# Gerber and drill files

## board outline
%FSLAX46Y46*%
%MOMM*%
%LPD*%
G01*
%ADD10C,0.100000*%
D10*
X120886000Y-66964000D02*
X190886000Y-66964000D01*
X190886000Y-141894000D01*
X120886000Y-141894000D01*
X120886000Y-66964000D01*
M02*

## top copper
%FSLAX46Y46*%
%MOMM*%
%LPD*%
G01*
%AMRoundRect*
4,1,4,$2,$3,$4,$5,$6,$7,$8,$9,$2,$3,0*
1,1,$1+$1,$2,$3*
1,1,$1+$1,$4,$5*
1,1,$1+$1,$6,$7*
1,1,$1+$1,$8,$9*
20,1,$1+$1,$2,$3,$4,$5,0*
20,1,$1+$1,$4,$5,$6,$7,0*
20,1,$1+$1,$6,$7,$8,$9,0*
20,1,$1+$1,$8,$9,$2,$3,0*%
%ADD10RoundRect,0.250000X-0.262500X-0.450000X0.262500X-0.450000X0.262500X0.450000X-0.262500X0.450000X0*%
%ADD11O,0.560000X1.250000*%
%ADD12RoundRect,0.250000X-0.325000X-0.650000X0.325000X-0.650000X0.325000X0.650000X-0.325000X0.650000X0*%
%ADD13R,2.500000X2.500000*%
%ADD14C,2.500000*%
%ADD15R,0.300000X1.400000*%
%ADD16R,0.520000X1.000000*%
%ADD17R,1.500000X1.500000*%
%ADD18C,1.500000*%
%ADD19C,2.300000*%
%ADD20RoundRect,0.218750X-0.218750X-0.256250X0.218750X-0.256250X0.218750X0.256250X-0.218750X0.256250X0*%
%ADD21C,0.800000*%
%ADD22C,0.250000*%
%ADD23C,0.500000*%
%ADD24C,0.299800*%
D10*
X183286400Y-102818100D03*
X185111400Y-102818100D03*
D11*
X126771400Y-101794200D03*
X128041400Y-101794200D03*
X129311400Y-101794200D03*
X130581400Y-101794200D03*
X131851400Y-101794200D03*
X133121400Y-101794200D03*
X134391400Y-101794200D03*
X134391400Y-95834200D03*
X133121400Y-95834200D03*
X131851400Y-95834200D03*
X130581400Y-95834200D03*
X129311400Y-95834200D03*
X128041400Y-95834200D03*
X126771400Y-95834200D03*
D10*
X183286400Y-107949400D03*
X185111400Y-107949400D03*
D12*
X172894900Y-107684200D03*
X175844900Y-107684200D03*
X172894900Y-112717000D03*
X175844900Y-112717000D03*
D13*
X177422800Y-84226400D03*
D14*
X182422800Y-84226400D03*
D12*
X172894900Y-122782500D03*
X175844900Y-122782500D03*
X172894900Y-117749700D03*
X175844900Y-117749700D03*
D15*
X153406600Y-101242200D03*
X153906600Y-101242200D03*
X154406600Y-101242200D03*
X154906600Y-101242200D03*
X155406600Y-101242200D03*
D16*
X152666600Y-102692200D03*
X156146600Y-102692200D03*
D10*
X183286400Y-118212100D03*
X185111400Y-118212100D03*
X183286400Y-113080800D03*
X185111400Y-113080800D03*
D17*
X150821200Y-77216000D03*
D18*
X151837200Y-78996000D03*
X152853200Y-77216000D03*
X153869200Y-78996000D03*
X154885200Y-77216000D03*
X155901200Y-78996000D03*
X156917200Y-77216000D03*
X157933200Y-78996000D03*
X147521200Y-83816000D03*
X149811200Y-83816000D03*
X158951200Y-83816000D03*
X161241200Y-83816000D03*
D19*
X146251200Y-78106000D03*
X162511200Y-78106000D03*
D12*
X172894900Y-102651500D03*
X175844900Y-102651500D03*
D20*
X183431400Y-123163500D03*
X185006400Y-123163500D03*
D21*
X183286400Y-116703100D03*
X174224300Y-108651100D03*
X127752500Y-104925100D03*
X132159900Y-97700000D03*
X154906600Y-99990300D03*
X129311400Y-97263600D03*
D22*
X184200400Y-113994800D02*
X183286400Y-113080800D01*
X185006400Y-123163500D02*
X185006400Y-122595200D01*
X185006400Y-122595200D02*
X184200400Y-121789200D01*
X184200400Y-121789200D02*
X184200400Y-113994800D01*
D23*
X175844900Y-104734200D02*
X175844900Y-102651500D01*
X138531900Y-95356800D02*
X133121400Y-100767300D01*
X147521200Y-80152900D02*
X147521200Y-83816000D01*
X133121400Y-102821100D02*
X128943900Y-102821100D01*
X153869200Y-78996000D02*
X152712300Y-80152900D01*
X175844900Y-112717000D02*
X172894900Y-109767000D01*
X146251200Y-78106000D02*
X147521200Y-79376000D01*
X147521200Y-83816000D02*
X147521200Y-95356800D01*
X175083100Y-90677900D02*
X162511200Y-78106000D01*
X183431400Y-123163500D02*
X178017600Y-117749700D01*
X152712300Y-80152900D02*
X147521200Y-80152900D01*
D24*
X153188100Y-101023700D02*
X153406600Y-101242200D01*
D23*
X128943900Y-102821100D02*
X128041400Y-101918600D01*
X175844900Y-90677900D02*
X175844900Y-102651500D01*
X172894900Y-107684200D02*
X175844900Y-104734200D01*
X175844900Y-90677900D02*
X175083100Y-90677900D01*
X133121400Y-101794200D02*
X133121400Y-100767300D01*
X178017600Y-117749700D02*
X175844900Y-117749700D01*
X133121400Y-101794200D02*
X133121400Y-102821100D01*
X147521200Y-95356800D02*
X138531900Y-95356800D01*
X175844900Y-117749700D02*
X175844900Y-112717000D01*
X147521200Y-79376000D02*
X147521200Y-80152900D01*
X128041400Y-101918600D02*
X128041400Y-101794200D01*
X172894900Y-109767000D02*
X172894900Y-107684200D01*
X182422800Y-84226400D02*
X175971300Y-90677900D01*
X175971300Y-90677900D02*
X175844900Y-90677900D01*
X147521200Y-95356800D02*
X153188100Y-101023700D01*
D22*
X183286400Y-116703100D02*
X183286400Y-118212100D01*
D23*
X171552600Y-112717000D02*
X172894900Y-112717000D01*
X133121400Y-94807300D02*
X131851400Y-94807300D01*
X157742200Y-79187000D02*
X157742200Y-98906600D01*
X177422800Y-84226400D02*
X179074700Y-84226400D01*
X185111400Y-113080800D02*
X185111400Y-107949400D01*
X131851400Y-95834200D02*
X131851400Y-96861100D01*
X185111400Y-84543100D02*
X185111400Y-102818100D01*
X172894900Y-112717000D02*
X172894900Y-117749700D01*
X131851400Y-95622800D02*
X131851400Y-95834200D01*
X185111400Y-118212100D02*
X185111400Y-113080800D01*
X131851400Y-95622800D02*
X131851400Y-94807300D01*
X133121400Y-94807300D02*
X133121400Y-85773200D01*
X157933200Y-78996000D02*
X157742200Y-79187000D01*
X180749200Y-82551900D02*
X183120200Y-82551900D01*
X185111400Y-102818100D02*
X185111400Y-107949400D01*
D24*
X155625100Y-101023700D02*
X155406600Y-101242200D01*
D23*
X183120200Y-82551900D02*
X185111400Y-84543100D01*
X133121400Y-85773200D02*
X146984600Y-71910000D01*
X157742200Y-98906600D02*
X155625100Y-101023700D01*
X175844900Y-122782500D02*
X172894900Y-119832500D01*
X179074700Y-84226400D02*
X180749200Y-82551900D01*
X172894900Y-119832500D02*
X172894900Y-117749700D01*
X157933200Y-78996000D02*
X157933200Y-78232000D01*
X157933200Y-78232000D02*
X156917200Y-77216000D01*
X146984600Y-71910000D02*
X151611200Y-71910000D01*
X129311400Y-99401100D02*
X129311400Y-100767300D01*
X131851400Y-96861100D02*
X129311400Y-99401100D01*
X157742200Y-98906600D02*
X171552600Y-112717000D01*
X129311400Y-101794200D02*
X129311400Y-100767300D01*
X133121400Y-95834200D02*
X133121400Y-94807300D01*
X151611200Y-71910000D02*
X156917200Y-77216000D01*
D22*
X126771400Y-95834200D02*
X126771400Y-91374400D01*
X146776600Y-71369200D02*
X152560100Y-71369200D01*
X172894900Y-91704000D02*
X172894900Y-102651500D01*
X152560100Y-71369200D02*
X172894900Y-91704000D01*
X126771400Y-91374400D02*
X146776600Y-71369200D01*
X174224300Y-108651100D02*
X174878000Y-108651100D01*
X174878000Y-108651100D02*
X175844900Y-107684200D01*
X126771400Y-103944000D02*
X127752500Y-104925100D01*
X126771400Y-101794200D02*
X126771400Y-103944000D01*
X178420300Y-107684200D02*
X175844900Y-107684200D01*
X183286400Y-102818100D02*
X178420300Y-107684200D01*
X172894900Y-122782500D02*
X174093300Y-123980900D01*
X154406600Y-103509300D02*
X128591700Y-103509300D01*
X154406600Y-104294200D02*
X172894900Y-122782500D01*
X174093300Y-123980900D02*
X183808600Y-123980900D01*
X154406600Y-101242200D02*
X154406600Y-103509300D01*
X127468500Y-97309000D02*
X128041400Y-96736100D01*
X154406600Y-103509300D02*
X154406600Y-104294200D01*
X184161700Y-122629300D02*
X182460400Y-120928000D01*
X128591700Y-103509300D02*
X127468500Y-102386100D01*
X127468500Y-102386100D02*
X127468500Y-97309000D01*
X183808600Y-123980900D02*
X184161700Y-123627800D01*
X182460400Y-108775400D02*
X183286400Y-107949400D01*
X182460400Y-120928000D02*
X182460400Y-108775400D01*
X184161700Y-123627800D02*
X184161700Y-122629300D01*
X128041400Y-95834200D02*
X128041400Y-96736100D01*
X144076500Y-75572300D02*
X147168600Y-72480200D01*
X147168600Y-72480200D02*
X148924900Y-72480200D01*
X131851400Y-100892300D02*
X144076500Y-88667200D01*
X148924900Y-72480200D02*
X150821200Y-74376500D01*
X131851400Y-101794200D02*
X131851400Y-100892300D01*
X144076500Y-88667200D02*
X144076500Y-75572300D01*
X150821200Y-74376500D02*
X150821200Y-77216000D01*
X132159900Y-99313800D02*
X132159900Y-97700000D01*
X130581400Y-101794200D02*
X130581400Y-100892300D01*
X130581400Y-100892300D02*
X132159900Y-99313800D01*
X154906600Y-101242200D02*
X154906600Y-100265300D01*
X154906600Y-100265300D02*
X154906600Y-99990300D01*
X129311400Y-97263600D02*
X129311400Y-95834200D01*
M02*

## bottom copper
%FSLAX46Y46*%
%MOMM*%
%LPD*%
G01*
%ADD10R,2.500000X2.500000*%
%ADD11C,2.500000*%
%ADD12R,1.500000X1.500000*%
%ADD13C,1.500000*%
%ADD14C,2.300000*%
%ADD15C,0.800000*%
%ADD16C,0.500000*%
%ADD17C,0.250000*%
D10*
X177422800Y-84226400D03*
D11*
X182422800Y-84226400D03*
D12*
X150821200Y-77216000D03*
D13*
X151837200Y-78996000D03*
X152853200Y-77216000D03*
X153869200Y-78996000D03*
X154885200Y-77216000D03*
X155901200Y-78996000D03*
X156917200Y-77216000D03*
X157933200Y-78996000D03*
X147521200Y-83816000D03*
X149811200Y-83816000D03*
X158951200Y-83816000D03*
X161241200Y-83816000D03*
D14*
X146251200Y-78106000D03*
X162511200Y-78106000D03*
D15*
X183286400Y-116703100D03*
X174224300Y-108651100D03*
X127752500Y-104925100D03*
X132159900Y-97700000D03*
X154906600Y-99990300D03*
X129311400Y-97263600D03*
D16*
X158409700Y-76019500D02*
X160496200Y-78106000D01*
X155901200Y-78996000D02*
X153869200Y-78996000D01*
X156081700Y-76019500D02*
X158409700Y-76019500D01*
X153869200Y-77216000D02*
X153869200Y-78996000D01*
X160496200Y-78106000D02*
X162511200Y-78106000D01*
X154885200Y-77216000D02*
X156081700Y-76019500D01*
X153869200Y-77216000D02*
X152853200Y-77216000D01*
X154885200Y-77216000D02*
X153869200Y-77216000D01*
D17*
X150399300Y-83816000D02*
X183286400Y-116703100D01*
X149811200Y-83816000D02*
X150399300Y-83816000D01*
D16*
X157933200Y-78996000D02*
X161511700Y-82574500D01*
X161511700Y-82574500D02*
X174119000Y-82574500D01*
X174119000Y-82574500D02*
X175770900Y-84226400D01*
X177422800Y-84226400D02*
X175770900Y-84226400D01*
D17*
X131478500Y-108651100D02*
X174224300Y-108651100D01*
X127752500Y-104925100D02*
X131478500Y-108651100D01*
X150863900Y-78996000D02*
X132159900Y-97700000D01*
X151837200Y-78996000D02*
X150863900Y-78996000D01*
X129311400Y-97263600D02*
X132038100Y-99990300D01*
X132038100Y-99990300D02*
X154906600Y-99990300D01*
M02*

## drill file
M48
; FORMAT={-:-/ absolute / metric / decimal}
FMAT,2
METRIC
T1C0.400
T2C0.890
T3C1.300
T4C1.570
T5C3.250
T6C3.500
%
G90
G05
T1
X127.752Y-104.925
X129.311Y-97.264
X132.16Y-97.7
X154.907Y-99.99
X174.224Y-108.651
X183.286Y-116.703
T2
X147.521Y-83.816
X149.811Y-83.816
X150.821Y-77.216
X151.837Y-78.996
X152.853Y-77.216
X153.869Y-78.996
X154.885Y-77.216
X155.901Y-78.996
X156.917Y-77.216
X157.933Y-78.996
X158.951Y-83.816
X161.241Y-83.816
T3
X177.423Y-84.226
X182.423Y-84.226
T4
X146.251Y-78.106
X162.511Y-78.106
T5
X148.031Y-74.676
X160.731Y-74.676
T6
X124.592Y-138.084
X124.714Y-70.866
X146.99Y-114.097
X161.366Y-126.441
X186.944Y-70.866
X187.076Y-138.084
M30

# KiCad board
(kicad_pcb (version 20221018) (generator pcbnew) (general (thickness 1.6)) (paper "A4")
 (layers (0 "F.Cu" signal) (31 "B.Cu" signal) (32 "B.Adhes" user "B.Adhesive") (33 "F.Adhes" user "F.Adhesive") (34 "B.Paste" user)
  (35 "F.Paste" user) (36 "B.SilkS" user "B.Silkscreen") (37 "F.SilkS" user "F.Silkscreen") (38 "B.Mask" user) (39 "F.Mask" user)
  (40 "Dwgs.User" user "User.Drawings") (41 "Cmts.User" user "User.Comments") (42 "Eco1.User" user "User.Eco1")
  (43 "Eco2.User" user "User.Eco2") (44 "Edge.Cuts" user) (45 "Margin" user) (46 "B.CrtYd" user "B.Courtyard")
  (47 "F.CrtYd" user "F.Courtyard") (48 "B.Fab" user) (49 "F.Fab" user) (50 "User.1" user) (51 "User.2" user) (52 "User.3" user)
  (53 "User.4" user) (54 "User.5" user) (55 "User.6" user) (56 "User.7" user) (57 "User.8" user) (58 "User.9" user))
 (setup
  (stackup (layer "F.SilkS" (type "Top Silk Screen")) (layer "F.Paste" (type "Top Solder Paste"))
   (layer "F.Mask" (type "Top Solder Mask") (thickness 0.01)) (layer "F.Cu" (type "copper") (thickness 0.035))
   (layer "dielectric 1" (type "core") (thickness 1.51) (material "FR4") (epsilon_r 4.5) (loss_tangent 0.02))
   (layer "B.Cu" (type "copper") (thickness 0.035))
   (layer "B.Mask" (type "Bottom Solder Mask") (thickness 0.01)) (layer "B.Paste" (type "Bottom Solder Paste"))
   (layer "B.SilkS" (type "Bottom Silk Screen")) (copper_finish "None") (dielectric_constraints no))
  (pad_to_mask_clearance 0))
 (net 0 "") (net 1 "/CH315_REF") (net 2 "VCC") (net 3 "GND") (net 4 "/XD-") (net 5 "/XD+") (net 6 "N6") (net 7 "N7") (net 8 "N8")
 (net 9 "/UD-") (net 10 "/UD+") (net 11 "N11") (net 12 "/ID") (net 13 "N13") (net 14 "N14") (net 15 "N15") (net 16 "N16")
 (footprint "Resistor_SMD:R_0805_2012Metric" (layer "F.Cu") (at 184.1989 102.8181)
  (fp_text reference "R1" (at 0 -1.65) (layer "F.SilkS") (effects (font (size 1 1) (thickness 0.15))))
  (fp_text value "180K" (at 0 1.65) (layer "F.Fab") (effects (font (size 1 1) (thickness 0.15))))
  (pad "1" smd roundrect (at -0.9125 0) (size 1.025 1.4) (layers "F.Cu" "F.Paste" "F.Mask") (roundrect_rratio 0.243902439)
   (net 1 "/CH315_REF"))
  (pad "2" smd roundrect (at 0.9125 0) (size 1.025 1.4) (layers "F.Cu" "F.Paste" "F.Mask") (roundrect_rratio 0.243902439) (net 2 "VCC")))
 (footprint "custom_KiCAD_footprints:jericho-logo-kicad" (layer "F.Cu") (at 154.813 79.5274)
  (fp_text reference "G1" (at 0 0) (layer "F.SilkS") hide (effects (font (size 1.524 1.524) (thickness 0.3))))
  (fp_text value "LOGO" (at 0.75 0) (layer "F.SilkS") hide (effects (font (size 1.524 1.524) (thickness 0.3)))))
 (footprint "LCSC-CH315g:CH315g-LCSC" (layer "F.Cu") (at 130.5814 98.8142)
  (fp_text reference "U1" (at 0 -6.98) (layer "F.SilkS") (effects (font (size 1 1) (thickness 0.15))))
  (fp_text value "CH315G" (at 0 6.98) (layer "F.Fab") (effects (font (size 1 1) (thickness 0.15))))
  (pad "1" smd oval (at -3.81 2.98) (size 0.56 1.25) (layers "F.Cu" "F.Paste" "F.Mask") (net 1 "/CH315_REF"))
  (pad "2" smd oval (at -2.54 2.98) (size 0.56 1.25) (layers "F.Cu" "F.Paste" "F.Mask") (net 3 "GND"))
  (pad "3" smd oval (at -1.27 2.98) (size 0.56 1.25) (layers "F.Cu" "F.Paste" "F.Mask") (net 2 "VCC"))
  (pad "4" smd oval (at 0 2.98) (size 0.56 1.25) (layers "F.Cu" "F.Paste" "F.Mask") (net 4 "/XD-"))
  (pad "5" smd oval (at 1.27 2.98) (size 0.56 1.25) (layers "F.Cu" "F.Paste" "F.Mask") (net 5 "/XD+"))
  (pad "6" smd oval (at 2.54 2.98) (size 0.56 1.25) (layers "F.Cu" "F.Paste" "F.Mask") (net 3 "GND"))
  (pad "7" smd oval (at 3.81 2.98) (size 0.56 1.25) (layers "F.Cu" "F.Paste" "F.Mask") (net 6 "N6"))
  (pad "8" smd oval (at 3.81 -2.98) (size 0.56 1.25) (layers "F.Cu" "F.Paste" "F.Mask") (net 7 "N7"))
  (pad "9" smd oval (at 2.54 -2.98) (size 0.56 1.25) (layers "F.Cu" "F.Paste" "F.Mask") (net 2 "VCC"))
  (pad "10" smd oval (at 1.27 -2.98) (size 0.56 1.25) (layers "F.Cu" "F.Paste" "F.Mask") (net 2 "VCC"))
  (pad "11" smd oval (at 0 -2.98) (size 0.56 1.25) (layers "F.Cu" "F.Paste" "F.Mask") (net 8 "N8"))
  (pad "12" smd oval (at -1.27 -2.98) (size 0.56 1.25) (layers "F.Cu" "F.Paste" "F.Mask") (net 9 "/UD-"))
  (pad "13" smd oval (at -2.54 -2.98) (size 0.56 1.25) (layers "F.Cu" "F.Paste" "F.Mask") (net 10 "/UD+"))
  (pad "14" smd oval (at -3.81 -2.98) (size 0.56 1.25) (layers "F.Cu" "F.Paste" "F.Mask") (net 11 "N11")))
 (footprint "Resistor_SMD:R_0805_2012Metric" (layer "F.Cu") (at 184.1989 107.9494)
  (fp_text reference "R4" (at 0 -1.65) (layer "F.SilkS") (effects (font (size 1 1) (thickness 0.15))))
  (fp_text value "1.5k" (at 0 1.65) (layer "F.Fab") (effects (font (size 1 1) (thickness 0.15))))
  (pad "1" smd roundrect (at -0.9125 0) (size 1.025 1.4) (layers "F.Cu" "F.Paste" "F.Mask") (roundrect_rratio 0.243902439) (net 10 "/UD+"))
  (pad "2" smd roundrect (at 0.9125 0) (size 1.025 1.4) (layers "F.Cu" "F.Paste" "F.Mask") (roundrect_rratio 0.243902439) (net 2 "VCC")))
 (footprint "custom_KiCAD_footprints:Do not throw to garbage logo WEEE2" (layer "F.Cu") (at 156.337 117.3734 90)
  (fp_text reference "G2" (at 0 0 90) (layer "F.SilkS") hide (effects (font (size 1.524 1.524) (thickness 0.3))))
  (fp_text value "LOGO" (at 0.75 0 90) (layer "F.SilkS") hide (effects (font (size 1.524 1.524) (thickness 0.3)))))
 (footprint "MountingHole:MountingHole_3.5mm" (layer "F.Cu") (at 186.944 70.866)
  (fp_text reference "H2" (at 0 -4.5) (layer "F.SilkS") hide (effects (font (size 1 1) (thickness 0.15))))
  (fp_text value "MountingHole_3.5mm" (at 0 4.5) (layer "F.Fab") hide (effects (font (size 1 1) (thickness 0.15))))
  (pad "" np_thru_hole circle (at 0 0) (size 3.5 3.5) (drill 3.5) (layers "*.Cu" "*.Mask")))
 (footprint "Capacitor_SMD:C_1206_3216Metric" (layer "F.Cu") (at 174.3699 107.6842)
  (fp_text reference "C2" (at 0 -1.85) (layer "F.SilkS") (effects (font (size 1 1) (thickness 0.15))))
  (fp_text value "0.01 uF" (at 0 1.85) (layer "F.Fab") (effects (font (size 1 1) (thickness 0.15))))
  (pad "1" smd roundrect (at -1.475 0) (size 1.15 1.8) (layers "F.Cu" "F.Paste" "F.Mask") (roundrect_rratio 0.2173913043) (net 3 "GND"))
  (pad "2" smd roundrect (at 1.475 0) (size 1.15 1.8) (layers "F.Cu" "F.Paste" "F.Mask") (roundrect_rratio 0.2173913043)
   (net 1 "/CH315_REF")))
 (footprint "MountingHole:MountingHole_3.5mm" (layer "F.Cu") (at 146.9898 114.0968)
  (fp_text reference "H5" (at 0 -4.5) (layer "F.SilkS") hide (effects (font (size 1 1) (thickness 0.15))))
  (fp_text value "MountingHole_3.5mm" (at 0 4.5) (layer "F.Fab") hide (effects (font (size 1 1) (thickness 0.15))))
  (pad "" np_thru_hole circle (at 0 0) (size 3.5 3.5) (drill 3.5) (layers "F&B.Cu" "*.Mask")))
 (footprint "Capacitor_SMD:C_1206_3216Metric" (layer "F.Cu") (at 174.3699 112.717)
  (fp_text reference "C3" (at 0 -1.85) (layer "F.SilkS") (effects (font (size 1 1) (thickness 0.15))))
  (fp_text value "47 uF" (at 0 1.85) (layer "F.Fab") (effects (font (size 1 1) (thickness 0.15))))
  (pad "1" smd roundrect (at -1.475 0) (size 1.15 1.8) (layers "F.Cu" "F.Paste" "F.Mask") (roundrect_rratio 0.2173913043) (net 2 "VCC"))
  (pad "2" smd roundrect (at 1.475 0) (size 1.15 1.8) (layers "F.Cu" "F.Paste" "F.Mask") (roundrect_rratio 0.2173913043) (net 3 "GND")))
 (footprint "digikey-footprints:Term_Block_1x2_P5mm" (layer "F.Cu") (at 177.4228 84.2264)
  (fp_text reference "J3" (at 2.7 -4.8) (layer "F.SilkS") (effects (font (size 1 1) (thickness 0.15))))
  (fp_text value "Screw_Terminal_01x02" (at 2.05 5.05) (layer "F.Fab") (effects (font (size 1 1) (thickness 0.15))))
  (pad "1" thru_hole rect (at 0 0) (size 2.5 2.5) (drill 1.3) (layers "*.Cu" "*.Mask") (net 2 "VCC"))
  (pad "2" thru_hole circle (at 5 0) (size 2.5 2.5) (drill 1.3) (layers "*.Cu" "*.Mask") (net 3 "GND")))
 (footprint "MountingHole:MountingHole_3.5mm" (layer "F.Cu") (at 187.076 138.084 -90)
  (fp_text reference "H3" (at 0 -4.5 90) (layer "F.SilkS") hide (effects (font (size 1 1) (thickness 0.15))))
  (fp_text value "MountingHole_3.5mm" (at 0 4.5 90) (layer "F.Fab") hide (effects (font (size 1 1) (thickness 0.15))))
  (pad "" np_thru_hole circle (at 0 0 270) (size 3.5 3.5) (drill 3.5) (layers "*.Cu" "*.Mask")))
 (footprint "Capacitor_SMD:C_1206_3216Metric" (layer "F.Cu") (at 174.3699 122.7825)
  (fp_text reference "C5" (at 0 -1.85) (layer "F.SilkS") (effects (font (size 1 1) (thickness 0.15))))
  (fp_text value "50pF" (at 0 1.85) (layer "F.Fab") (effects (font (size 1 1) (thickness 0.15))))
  (pad "1" smd roundrect (at -1.475 0) (size 1.15 1.8) (layers "F.Cu" "F.Paste" "F.Mask") (roundrect_rratio 0.2173913043) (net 10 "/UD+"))
  (pad "2" smd roundrect (at 1.475 0) (size 1.15 1.8) (layers "F.Cu" "F.Paste" "F.Mask") (roundrect_rratio 0.2173913043) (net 2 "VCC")))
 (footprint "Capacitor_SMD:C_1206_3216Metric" (layer "F.Cu") (at 174.3699 117.7497)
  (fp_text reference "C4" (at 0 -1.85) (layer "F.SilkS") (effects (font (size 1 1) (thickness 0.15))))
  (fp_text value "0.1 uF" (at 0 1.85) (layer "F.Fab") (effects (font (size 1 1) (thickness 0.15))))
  (pad "1" smd roundrect (at -1.475 0) (size 1.15 1.8) (layers "F.Cu" "F.Paste" "F.Mask") (roundrect_rratio 0.2173913043) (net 2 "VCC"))
  (pad "2" smd roundrect (at 1.475 0) (size 1.15 1.8) (layers "F.Cu" "F.Paste" "F.Mask") (roundrect_rratio 0.2173913043) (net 3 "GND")))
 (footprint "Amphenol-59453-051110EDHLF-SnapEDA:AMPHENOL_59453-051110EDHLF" (layer "F.Cu") (at 154.4066 102.6922)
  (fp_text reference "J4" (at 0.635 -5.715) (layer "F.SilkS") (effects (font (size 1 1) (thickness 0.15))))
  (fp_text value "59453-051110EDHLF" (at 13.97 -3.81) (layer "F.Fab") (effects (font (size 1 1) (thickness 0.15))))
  (pad "1" smd rect (at -1 -1.45) (size 0.3 1.4) (layers "F.Cu" "F.Paste" "F.Mask") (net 3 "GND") (solder_mask_margin 0.102))
  (pad "2" smd rect (at -0.5 -1.45) (size 0.3 1.4) (layers "F.Cu" "F.Paste" "F.Mask") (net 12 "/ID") (solder_mask_margin 0.102))
  (pad "3" smd rect (at 0 -1.45) (size 0.3 1.4) (layers "F.Cu" "F.Paste" "F.Mask") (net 10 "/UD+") (solder_mask_margin 0.102))
  (pad "4" smd rect (at 0.5 -1.45) (size 0.3 1.4) (layers "F.Cu" "F.Paste" "F.Mask") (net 9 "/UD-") (solder_mask_margin 0.102))
  (pad "5" smd rect (at 1 -1.45) (size 0.3 1.4) (layers "F.Cu" "F.Paste" "F.Mask") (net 2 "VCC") (solder_mask_margin 0.102))
  (pad "S1" smd rect (at -1.74 0) (size 0.52 1) (layers "F.Cu" "F.Paste" "F.Mask") (solder_mask_margin 0.102))
  (pad "S2" smd rect (at 1.74 0) (size 0.52 1) (layers "F.Cu" "F.Paste" "F.Mask") (solder_mask_margin 0.102)))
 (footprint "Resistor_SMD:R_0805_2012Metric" (layer "F.Cu") (at 184.1989 118.2121)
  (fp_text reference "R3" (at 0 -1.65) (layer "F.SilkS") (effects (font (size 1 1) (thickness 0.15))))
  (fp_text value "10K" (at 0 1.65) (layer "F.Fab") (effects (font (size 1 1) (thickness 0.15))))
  (pad "1" smd roundrect (at -0.9125 0) (size 1.025 1.4) (layers "F.Cu" "F.Paste" "F.Mask") (roundrect_rratio 0.243902439) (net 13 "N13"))
  (pad "2" smd roundrect (at 0.9125 0) (size 1.025 1.4) (layers "F.Cu" "F.Paste" "F.Mask") (roundrect_rratio 0.243902439) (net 2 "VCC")))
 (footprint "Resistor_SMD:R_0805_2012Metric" (layer "F.Cu") (at 184.1989 113.0808)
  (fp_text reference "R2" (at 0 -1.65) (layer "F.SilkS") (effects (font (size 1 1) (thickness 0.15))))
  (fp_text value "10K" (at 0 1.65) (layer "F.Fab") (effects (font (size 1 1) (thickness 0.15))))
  (pad "1" smd roundrect (at -0.9125 0) (size 1.025 1.4) (layers "F.Cu" "F.Paste" "F.Mask") (roundrect_rratio 0.243902439) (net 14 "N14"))
  (pad "2" smd roundrect (at 0.9125 0) (size 1.025 1.4) (layers "F.Cu" "F.Paste" "F.Mask") (roundrect_rratio 0.243902439) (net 2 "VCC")))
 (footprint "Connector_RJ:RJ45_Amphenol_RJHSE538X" (layer "F.Cu") (at 150.8212 77.216)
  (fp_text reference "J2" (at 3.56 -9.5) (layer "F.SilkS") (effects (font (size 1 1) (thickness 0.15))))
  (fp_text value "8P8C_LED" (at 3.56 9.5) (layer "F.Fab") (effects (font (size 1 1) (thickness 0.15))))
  (pad "" np_thru_hole circle (at -2.79 -2.54) (size 3.25 3.25) (drill 3.25) (layers "*.Cu" "*.Mask"))
  (pad "" np_thru_hole circle (at 9.91 -2.54) (size 3.25 3.25) (drill 3.25) (layers "*.Cu" "*.Mask"))
  (pad "1" thru_hole rect (at 0 0) (size 1.5 1.5) (drill 0.89) (layers "*.Cu" "*.Mask") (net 5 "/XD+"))
  (pad "2" thru_hole circle (at 1.016 1.78) (size 1.5 1.5) (drill 0.89) (layers "*.Cu" "*.Mask") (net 4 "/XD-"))
  (pad "3" thru_hole circle (at 2.032 0) (size 1.5 1.5) (drill 0.89) (layers "*.Cu" "*.Mask") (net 3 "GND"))
  (pad "4" thru_hole circle (at 3.048 1.78) (size 1.5 1.5) (drill 0.89) (layers "*.Cu" "*.Mask") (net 3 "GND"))
  (pad "5" thru_hole circle (at 4.064 0) (size 1.5 1.5) (drill 0.89) (layers "*.Cu" "*.Mask") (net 3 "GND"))
  (pad "6" thru_hole circle (at 5.08 1.78) (size 1.5 1.5) (drill 0.89) (layers "*.Cu" "*.Mask") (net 3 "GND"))
  (pad "7" thru_hole circle (at 6.096 0) (size 1.5 1.5) (drill 0.89) (layers "*.Cu" "*.Mask") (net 2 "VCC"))
  (pad "8" thru_hole circle (at 7.112 1.78) (size 1.5 1.5) (drill 0.89) (layers "*.Cu" "*.Mask") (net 2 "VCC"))
  (pad "9" thru_hole circle (at -3.3 6.6) (size 1.5 1.5) (drill 0.89) (layers "*.Cu" "*.Mask") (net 3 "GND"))
  (pad "10" thru_hole circle (at -1.01 6.6) (size 1.5 1.5) (drill 0.89) (layers "*.Cu" "*.Mask") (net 13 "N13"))
  (pad "11" thru_hole circle (at 8.13 6.6) (size 1.5 1.5) (drill 0.89) (layers "*.Cu" "*.Mask") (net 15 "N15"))
  (pad "12" thru_hole circle (at 10.42 6.6) (size 1.5 1.5) (drill 0.89) (layers "*.Cu" "*.Mask") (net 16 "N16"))
  (pad "SH" thru_hole circle (at -4.57 0.89) (size 2.3 2.3) (drill 1.57) (layers "*.Cu" "*.Mask") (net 3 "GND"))
  (pad "SH" thru_hole circle (at 11.69 0.89) (size 2.3 2.3) (drill 1.57) (layers "*.Cu" "*.Mask") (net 3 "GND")))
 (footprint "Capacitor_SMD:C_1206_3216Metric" (layer "F.Cu") (at 174.3699 102.6515)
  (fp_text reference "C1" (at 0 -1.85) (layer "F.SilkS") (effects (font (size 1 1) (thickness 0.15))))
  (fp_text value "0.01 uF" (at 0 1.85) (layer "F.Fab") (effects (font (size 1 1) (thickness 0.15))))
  (pad "1" smd roundrect (at -1.475 0) (size 1.15 1.8) (layers "F.Cu" "F.Paste" "F.Mask") (roundrect_rratio 0.2173913043) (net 11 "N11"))
  (pad "2" smd roundrect (at 1.475 0) (size 1.15 1.8) (layers "F.Cu" "F.Paste" "F.Mask") (roundrect_rratio 0.2173913043) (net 3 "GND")))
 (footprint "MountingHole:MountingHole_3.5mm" (layer "F.Cu") (at 124.714 70.866 90)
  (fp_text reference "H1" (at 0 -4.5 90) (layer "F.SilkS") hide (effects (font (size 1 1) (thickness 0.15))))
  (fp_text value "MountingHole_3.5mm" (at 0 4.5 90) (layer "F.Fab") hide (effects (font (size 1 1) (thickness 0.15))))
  (pad "" np_thru_hole circle (at 0 0 90) (size 3.5 3.5) (drill 3.5) (layers "*.Cu" "*.Mask")))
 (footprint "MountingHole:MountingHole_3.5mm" (layer "F.Cu") (at 161.3662 126.4412 -90)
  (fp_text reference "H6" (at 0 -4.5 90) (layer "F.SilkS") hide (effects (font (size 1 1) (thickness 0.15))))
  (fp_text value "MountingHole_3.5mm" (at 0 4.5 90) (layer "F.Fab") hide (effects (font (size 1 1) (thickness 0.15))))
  (pad "" np_thru_hole circle (at 0 0 270) (size 3.5 3.5) (drill 3.5) (layers "F&B.Cu" "*.Mask")))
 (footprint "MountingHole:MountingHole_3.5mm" (layer "F.Cu") (at 124.592 138.084 180)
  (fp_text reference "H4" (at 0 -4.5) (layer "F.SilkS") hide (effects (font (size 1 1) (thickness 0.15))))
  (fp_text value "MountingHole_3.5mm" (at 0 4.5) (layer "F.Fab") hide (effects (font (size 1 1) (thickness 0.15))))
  (pad "" np_thru_hole circle (at 0 0 180) (size 3.5 3.5) (drill 3.5) (layers "*.Cu" "*.Mask")))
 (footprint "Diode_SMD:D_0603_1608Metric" (layer "F.Cu") (at 184.2189 123.1635)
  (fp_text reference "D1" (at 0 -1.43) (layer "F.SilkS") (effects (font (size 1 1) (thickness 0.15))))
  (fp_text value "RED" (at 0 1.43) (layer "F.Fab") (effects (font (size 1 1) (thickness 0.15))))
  (pad "1" smd roundrect (at -0.7875 0) (size 0.875 0.95) (layers "F.Cu" "F.Paste" "F.Mask") (roundrect_rratio 0.25) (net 3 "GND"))
  (pad "2" smd roundrect (at 0.7875 0) (size 0.875 0.95) (layers "F.Cu" "F.Paste" "F.Mask") (roundrect_rratio 0.25) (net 14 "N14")))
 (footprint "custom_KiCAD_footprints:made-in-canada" (layer "B.Cu") (at 155.321 99.8474 180)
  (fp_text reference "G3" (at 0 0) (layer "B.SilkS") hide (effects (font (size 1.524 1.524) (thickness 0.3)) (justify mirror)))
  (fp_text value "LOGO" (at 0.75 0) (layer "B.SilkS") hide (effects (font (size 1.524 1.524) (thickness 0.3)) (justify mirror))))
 (gr_rect (start 120.886 66.964) (end 190.886 141.894) (stroke (width 0.1) (type default)) (fill none) (layer "Edge.Cuts"))
 (segment (start 184.2004 113.9948) (end 183.2864 113.0808) (width 0.25) (layer "F.Cu") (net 14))
 (segment (start 185.0064 123.1635) (end 185.0064 122.5952) (width 0.25) (layer "F.Cu") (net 14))
 (segment (start 185.0064 122.5952) (end 184.2004 121.7892) (width 0.25) (layer "F.Cu") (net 14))
 (segment (start 184.2004 121.7892) (end 184.2004 113.9948) (width 0.25) (layer "F.Cu") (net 14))
 (segment (start 175.8449 104.7342) (end 175.8449 102.6515) (width 0.5) (layer "F.Cu") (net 3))
 (segment (start 138.5319 95.3568) (end 133.1214 100.7673) (width 0.5) (layer "F.Cu") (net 3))
 (segment (start 147.5212 80.1529) (end 147.5212 83.816) (width 0.5) (layer "F.Cu") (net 3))
 (segment (start 133.1214 102.8211) (end 128.9439 102.8211) (width 0.5) (layer "F.Cu") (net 3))
 (segment (start 153.8692 78.996) (end 152.7123 80.1529) (width 0.5) (layer "F.Cu") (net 3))
 (segment (start 175.8449 112.717) (end 172.8949 109.767) (width 0.5) (layer "F.Cu") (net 3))
 (segment (start 146.2512 78.106) (end 147.5212 79.376) (width 0.5) (layer "F.Cu") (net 3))
 (segment (start 147.5212 83.816) (end 147.5212 95.3568) (width 0.5) (layer "F.Cu") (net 3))
 (segment (start 175.0831 90.6779) (end 162.5112 78.106) (width 0.5) (layer "F.Cu") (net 3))
 (segment (start 183.4314 123.1635) (end 178.0176 117.7497) (width 0.5) (layer "F.Cu") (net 3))
 (segment (start 152.7123 80.1529) (end 147.5212 80.1529) (width 0.5) (layer "F.Cu") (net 3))
 (segment (start 153.1881 101.0237) (end 153.4066 101.2422) (width 0.2998) (layer "F.Cu") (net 3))
 (segment (start 128.9439 102.8211) (end 128.0414 101.9186) (width 0.5) (layer "F.Cu") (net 3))
 (segment (start 175.8449 90.6779) (end 175.8449 102.6515) (width 0.5) (layer "F.Cu") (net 3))
 (segment (start 172.8949 107.6842) (end 175.8449 104.7342) (width 0.5) (layer "F.Cu") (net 3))
 (segment (start 175.8449 90.6779) (end 175.0831 90.6779) (width 0.5) (layer "F.Cu") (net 3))
 (segment (start 133.1214 101.7942) (end 133.1214 100.7673) (width 0.5) (layer "F.Cu") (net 3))
 (segment (start 178.0176 117.7497) (end 175.8449 117.7497) (width 0.5) (layer "F.Cu") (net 3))
 (segment (start 133.1214 101.7942) (end 133.1214 102.8211) (width 0.5) (layer "F.Cu") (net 3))
 (segment (start 147.5212 95.3568) (end 138.5319 95.3568) (width 0.5) (layer "F.Cu") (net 3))
 (segment (start 175.8449 117.7497) (end 175.8449 112.717) (width 0.5) (layer "F.Cu") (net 3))
 (segment (start 147.5212 79.376) (end 147.5212 80.1529) (width 0.5) (layer "F.Cu") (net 3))
 (segment (start 128.0414 101.9186) (end 128.0414 101.7942) (width 0.5) (layer "F.Cu") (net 3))
 (segment (start 172.8949 109.767) (end 172.8949 107.6842) (width 0.5) (layer "F.Cu") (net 3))
 (segment (start 182.4228 84.2264) (end 175.9713 90.6779) (width 0.5) (layer "F.Cu") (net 3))
 (segment (start 175.9713 90.6779) (end 175.8449 90.6779) (width 0.5) (layer "F.Cu") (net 3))
 (segment (start 147.5212 95.3568) (end 153.1881 101.0237) (width 0.5) (layer "F.Cu") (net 3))
 (segment (start 158.4097 76.0195) (end 160.4962 78.106) (width 0.5) (layer "B.Cu") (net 3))
 (segment (start 155.9012 78.996) (end 153.8692 78.996) (width 0.5) (layer "B.Cu") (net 3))
 (segment (start 156.0817 76.0195) (end 158.4097 76.0195) (width 0.5) (layer "B.Cu") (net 3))
 (segment (start 153.8692 77.216) (end 153.8692 78.996) (width 0.5) (layer "B.Cu") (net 3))
 (segment (start 160.4962 78.106) (end 162.5112 78.106) (width 0.5) (layer "B.Cu") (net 3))
 (segment (start 154.8852 77.216) (end 156.0817 76.0195) (width 0.5) (layer "B.Cu") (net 3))
 (segment (start 153.8692 77.216) (end 152.8532 77.216) (width 0.5) (layer "B.Cu") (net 3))
 (segment (start 154.8852 77.216) (end 153.8692 77.216) (width 0.5) (layer "B.Cu") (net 3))
 (segment (start 183.2864 116.7031) (end 183.2864 118.2121) (width 0.25) (layer "F.Cu") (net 13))
 (via (at 183.2864 116.7031) (size 0.8) (drill 0.4) (layers "F.Cu" "B.Cu") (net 13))
 (segment (start 150.3993 83.816) (end 183.2864 116.7031) (width 0.25) (layer "B.Cu") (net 13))
 (segment (start 149.8112 83.816) (end 150.3993 83.816) (width 0.25) (layer "B.Cu") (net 13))
 (segment (start 171.5526 112.717) (end 172.8949 112.717) (width 0.5) (layer "F.Cu") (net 2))
 (segment (start 133.1214 94.8073) (end 131.8514 94.8073) (width 0.5) (layer "F.Cu") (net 2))
 (segment (start 157.7422 79.187) (end 157.7422 98.9066) (width 0.5) (layer "F.Cu") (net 2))
 (segment (start 177.4228 84.2264) (end 179.0747 84.2264) (width 0.5) (layer "F.Cu") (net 2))
 (segment (start 185.1114 113.0808) (end 185.1114 107.9494) (width 0.5) (layer "F.Cu") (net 2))
 (segment (start 131.8514 95.8342) (end 131.8514 96.8611) (width 0.5) (layer "F.Cu") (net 2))
 (segment (start 185.1114 84.5431) (end 185.1114 102.8181) (width 0.5) (layer "F.Cu") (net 2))
 (segment (start 172.8949 112.717) (end 172.8949 117.7497) (width 0.5) (layer "F.Cu") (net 2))
 (segment (start 131.8514 95.6228) (end 131.8514 95.8342) (width 0.5) (layer "F.Cu") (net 2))
 (segment (start 185.1114 118.2121) (end 185.1114 113.0808) (width 0.5) (layer "F.Cu") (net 2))
 (segment (start 131.8514 95.6228) (end 131.8514 94.8073) (width 0.5) (layer "F.Cu") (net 2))
 (segment (start 133.1214 94.8073) (end 133.1214 85.7732) (width 0.5) (layer "F.Cu") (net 2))
 (segment (start 157.9332 78.996) (end 157.7422 79.187) (width 0.5) (layer "F.Cu") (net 2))
 (segment (start 180.7492 82.5519) (end 183.1202 82.5519) (width 0.5) (layer "F.Cu") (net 2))
 (segment (start 185.1114 102.8181) (end 185.1114 107.9494) (width 0.5) (layer "F.Cu") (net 2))
 (segment (start 155.6251 101.0237) (end 155.4066 101.2422) (width 0.2998) (layer "F.Cu") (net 2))
 (segment (start 183.1202 82.5519) (end 185.1114 84.5431) (width 0.5) (layer "F.Cu") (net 2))
 (segment (start 133.1214 85.7732) (end 146.9846 71.91) (width 0.5) (layer "F.Cu") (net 2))
 (segment (start 157.7422 98.9066) (end 155.6251 101.0237) (width 0.5) (layer "F.Cu") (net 2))
 (segment (start 175.8449 122.7825) (end 172.8949 119.8325) (width 0.5) (layer "F.Cu") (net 2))
 (segment (start 179.0747 84.2264) (end 180.7492 82.5519) (width 0.5) (layer "F.Cu") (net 2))
 (segment (start 172.8949 119.8325) (end 172.8949 117.7497) (width 0.5) (layer "F.Cu") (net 2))
 (segment (start 157.9332 78.996) (end 157.9332 78.232) (width 0.5) (layer "F.Cu") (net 2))
 (segment (start 157.9332 78.232) (end 156.9172 77.216) (width 0.5) (layer "F.Cu") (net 2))
 (segment (start 146.9846 71.91) (end 151.6112 71.91) (width 0.5) (layer "F.Cu") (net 2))
 (segment (start 129.3114 99.4011) (end 129.3114 100.7673) (width 0.5) (layer "F.Cu") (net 2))
 (segment (start 131.8514 96.8611) (end 129.3114 99.4011) (width 0.5) (layer "F.Cu") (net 2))
 (segment (start 157.7422 98.9066) (end 171.5526 112.717) (width 0.5) (layer "F.Cu") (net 2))
 (segment (start 129.3114 101.7942) (end 129.3114 100.7673) (width 0.5) (layer "F.Cu") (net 2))
 (segment (start 133.1214 95.8342) (end 133.1214 94.8073) (width 0.5) (layer "F.Cu") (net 2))
 (segment (start 151.6112 71.91) (end 156.9172 77.216) (width 0.5) (layer "F.Cu") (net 2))
 (segment (start 157.9332 78.996) (end 161.5117 82.5745) (width 0.5) (layer "B.Cu") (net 2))
 (segment (start 161.5117 82.5745) (end 174.119 82.5745) (width 0.5) (layer "B.Cu") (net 2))
 (segment (start 174.119 82.5745) (end 175.7709 84.2264) (width 0.5) (layer "B.Cu") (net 2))
 (segment (start 177.4228 84.2264) (end 175.7709 84.2264) (width 0.5) (layer "B.Cu") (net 2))
 (segment (start 126.7714 95.8342) (end 126.7714 91.3744) (width 0.25) (layer "F.Cu") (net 11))
 (segment (start 146.7766 71.3692) (end 152.5601 71.3692) (width 0.25) (layer "F.Cu") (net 11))
 (segment (start 172.8949 91.704) (end 172.8949 102.6515) (width 0.25) (layer "F.Cu") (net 11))
 (segment (start 152.5601 71.3692) (end 172.8949 91.704) (width 0.25) (layer "F.Cu") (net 11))
 (segment (start 126.7714 91.3744) (end 146.7766 71.3692) (width 0.25) (layer "F.Cu") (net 11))
 (segment (start 174.2243 108.6511) (end 174.878 108.6511) (width 0.25) (layer "F.Cu") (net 1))
 (segment (start 174.878 108.6511) (end 175.8449 107.6842) (width 0.25) (layer "F.Cu") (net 1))
 (segment (start 126.7714 103.944) (end 127.7525 104.9251) (width 0.25) (layer "F.Cu") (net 1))
 (segment (start 126.7714 101.7942) (end 126.7714 103.944) (width 0.25) (layer "F.Cu") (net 1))
 (segment (start 178.4203 107.6842) (end 175.8449 107.6842) (width 0.25) (layer "F.Cu") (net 1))
 (segment (start 183.2864 102.8181) (end 178.4203 107.6842) (width 0.25) (layer "F.Cu") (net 1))
 (via (at 174.2243 108.6511) (size 0.8) (drill 0.4) (layers "F.Cu" "B.Cu") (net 1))
 (via (at 127.7525 104.9251) (size 0.8) (drill 0.4) (layers "F.Cu" "B.Cu") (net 1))
 (segment (start 131.4785 108.6511) (end 174.2243 108.6511) (width 0.25) (layer "B.Cu") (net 1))
 (segment (start 127.7525 104.9251) (end 131.4785 108.6511) (width 0.25) (layer "B.Cu") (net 1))
 (segment (start 172.8949 122.7825) (end 174.0933 123.9809) (width 0.25) (layer "F.Cu") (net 10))
 (segment (start 154.4066 103.5093) (end 128.5917 103.5093) (width 0.25) (layer "F.Cu") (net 10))
 (segment (start 154.4066 104.2942) (end 172.8949 122.7825) (width 0.25) (layer "F.Cu") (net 10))
 (segment (start 174.0933 123.9809) (end 183.8086 123.9809) (width 0.25) (layer "F.Cu") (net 10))
 (segment (start 154.4066 101.2422) (end 154.4066 103.5093) (width 0.25) (layer "F.Cu") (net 10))
 (segment (start 127.4685 97.309) (end 128.0414 96.7361) (width 0.25) (layer "F.Cu") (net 10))
 (segment (start 154.4066 103.5093) (end 154.4066 104.2942) (width 0.25) (layer "F.Cu") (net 10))
 (segment (start 184.1617 122.6293) (end 182.4604 120.928) (width 0.25) (layer "F.Cu") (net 10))
 (segment (start 128.5917 103.5093) (end 127.4685 102.3861) (width 0.25) (layer "F.Cu") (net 10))
 (segment (start 127.4685 102.3861) (end 127.4685 97.309) (width 0.25) (layer "F.Cu") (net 10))
 (segment (start 183.8086 123.9809) (end 184.1617 123.6278) (width 0.25) (layer "F.Cu") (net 10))
 (segment (start 182.4604 108.7754) (end 183.2864 107.9494) (width 0.25) (layer "F.Cu") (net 10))
 (segment (start 182.4604 120.928) (end 182.4604 108.7754) (width 0.25) (layer "F.Cu") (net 10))
 (segment (start 184.1617 123.6278) (end 184.1617 122.6293) (width 0.25) (layer "F.Cu") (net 10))
 (segment (start 128.0414 95.8342) (end 128.0414 96.7361) (width 0.25) (layer "F.Cu") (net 10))
 (segment (start 144.0765 75.5723) (end 147.1686 72.4802) (width 0.25) (layer "F.Cu") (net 5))
 (segment (start 147.1686 72.4802) (end 148.9249 72.4802) (width 0.25) (layer "F.Cu") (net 5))
 (segment (start 131.8514 100.8923) (end 144.0765 88.6672) (width 0.25) (layer "F.Cu") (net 5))
 (segment (start 148.9249 72.4802) (end 150.8212 74.3765) (width 0.25) (layer "F.Cu") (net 5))
 (segment (start 131.8514 101.7942) (end 131.8514 100.8923) (width 0.25) (layer "F.Cu") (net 5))
 (segment (start 144.0765 88.6672) (end 144.0765 75.5723) (width 0.25) (layer "F.Cu") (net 5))
 (segment (start 150.8212 74.3765) (end 150.8212 77.216) (width 0.25) (layer "F.Cu") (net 5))
 (segment (start 132.1599 99.3138) (end 132.1599 97.7) (width 0.25) (layer "F.Cu") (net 4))
 (segment (start 130.5814 101.7942) (end 130.5814 100.8923) (width 0.25) (layer "F.Cu") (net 4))
 (segment (start 130.5814 100.8923) (end 132.1599 99.3138) (width 0.25) (layer "F.Cu") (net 4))
 (via (at 132.1599 97.7) (size 0.8) (drill 0.4) (layers "F.Cu" "B.Cu") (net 4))
 (segment (start 150.8639 78.996) (end 132.1599 97.7) (width 0.25) (layer "B.Cu") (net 4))
 (segment (start 151.8372 78.996) (end 150.8639 78.996) (width 0.25) (layer "B.Cu") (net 4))
 (segment (start 154.9066 101.2422) (end 154.9066 100.2653) (width 0.25) (layer "F.Cu") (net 9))
 (segment (start 154.9066 100.2653) (end 154.9066 99.9903) (width 0.25) (layer "F.Cu") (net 9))
 (segment (start 129.3114 97.2636) (end 129.3114 95.8342) (width 0.25) (layer "F.Cu") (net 9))
 (via (at 154.9066 99.9903) (size 0.8) (drill 0.4) (layers "F.Cu" "B.Cu") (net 9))
 (via (at 129.3114 97.2636) (size 0.8) (drill 0.4) (layers "F.Cu" "B.Cu") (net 9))
 (segment (start 129.3114 97.2636) (end 132.0381 99.9903) (width 0.25) (layer "B.Cu") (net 9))
 (segment (start 132.0381 99.9903) (end 154.9066 99.9903) (width 0.25) (layer "B.Cu") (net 9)))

